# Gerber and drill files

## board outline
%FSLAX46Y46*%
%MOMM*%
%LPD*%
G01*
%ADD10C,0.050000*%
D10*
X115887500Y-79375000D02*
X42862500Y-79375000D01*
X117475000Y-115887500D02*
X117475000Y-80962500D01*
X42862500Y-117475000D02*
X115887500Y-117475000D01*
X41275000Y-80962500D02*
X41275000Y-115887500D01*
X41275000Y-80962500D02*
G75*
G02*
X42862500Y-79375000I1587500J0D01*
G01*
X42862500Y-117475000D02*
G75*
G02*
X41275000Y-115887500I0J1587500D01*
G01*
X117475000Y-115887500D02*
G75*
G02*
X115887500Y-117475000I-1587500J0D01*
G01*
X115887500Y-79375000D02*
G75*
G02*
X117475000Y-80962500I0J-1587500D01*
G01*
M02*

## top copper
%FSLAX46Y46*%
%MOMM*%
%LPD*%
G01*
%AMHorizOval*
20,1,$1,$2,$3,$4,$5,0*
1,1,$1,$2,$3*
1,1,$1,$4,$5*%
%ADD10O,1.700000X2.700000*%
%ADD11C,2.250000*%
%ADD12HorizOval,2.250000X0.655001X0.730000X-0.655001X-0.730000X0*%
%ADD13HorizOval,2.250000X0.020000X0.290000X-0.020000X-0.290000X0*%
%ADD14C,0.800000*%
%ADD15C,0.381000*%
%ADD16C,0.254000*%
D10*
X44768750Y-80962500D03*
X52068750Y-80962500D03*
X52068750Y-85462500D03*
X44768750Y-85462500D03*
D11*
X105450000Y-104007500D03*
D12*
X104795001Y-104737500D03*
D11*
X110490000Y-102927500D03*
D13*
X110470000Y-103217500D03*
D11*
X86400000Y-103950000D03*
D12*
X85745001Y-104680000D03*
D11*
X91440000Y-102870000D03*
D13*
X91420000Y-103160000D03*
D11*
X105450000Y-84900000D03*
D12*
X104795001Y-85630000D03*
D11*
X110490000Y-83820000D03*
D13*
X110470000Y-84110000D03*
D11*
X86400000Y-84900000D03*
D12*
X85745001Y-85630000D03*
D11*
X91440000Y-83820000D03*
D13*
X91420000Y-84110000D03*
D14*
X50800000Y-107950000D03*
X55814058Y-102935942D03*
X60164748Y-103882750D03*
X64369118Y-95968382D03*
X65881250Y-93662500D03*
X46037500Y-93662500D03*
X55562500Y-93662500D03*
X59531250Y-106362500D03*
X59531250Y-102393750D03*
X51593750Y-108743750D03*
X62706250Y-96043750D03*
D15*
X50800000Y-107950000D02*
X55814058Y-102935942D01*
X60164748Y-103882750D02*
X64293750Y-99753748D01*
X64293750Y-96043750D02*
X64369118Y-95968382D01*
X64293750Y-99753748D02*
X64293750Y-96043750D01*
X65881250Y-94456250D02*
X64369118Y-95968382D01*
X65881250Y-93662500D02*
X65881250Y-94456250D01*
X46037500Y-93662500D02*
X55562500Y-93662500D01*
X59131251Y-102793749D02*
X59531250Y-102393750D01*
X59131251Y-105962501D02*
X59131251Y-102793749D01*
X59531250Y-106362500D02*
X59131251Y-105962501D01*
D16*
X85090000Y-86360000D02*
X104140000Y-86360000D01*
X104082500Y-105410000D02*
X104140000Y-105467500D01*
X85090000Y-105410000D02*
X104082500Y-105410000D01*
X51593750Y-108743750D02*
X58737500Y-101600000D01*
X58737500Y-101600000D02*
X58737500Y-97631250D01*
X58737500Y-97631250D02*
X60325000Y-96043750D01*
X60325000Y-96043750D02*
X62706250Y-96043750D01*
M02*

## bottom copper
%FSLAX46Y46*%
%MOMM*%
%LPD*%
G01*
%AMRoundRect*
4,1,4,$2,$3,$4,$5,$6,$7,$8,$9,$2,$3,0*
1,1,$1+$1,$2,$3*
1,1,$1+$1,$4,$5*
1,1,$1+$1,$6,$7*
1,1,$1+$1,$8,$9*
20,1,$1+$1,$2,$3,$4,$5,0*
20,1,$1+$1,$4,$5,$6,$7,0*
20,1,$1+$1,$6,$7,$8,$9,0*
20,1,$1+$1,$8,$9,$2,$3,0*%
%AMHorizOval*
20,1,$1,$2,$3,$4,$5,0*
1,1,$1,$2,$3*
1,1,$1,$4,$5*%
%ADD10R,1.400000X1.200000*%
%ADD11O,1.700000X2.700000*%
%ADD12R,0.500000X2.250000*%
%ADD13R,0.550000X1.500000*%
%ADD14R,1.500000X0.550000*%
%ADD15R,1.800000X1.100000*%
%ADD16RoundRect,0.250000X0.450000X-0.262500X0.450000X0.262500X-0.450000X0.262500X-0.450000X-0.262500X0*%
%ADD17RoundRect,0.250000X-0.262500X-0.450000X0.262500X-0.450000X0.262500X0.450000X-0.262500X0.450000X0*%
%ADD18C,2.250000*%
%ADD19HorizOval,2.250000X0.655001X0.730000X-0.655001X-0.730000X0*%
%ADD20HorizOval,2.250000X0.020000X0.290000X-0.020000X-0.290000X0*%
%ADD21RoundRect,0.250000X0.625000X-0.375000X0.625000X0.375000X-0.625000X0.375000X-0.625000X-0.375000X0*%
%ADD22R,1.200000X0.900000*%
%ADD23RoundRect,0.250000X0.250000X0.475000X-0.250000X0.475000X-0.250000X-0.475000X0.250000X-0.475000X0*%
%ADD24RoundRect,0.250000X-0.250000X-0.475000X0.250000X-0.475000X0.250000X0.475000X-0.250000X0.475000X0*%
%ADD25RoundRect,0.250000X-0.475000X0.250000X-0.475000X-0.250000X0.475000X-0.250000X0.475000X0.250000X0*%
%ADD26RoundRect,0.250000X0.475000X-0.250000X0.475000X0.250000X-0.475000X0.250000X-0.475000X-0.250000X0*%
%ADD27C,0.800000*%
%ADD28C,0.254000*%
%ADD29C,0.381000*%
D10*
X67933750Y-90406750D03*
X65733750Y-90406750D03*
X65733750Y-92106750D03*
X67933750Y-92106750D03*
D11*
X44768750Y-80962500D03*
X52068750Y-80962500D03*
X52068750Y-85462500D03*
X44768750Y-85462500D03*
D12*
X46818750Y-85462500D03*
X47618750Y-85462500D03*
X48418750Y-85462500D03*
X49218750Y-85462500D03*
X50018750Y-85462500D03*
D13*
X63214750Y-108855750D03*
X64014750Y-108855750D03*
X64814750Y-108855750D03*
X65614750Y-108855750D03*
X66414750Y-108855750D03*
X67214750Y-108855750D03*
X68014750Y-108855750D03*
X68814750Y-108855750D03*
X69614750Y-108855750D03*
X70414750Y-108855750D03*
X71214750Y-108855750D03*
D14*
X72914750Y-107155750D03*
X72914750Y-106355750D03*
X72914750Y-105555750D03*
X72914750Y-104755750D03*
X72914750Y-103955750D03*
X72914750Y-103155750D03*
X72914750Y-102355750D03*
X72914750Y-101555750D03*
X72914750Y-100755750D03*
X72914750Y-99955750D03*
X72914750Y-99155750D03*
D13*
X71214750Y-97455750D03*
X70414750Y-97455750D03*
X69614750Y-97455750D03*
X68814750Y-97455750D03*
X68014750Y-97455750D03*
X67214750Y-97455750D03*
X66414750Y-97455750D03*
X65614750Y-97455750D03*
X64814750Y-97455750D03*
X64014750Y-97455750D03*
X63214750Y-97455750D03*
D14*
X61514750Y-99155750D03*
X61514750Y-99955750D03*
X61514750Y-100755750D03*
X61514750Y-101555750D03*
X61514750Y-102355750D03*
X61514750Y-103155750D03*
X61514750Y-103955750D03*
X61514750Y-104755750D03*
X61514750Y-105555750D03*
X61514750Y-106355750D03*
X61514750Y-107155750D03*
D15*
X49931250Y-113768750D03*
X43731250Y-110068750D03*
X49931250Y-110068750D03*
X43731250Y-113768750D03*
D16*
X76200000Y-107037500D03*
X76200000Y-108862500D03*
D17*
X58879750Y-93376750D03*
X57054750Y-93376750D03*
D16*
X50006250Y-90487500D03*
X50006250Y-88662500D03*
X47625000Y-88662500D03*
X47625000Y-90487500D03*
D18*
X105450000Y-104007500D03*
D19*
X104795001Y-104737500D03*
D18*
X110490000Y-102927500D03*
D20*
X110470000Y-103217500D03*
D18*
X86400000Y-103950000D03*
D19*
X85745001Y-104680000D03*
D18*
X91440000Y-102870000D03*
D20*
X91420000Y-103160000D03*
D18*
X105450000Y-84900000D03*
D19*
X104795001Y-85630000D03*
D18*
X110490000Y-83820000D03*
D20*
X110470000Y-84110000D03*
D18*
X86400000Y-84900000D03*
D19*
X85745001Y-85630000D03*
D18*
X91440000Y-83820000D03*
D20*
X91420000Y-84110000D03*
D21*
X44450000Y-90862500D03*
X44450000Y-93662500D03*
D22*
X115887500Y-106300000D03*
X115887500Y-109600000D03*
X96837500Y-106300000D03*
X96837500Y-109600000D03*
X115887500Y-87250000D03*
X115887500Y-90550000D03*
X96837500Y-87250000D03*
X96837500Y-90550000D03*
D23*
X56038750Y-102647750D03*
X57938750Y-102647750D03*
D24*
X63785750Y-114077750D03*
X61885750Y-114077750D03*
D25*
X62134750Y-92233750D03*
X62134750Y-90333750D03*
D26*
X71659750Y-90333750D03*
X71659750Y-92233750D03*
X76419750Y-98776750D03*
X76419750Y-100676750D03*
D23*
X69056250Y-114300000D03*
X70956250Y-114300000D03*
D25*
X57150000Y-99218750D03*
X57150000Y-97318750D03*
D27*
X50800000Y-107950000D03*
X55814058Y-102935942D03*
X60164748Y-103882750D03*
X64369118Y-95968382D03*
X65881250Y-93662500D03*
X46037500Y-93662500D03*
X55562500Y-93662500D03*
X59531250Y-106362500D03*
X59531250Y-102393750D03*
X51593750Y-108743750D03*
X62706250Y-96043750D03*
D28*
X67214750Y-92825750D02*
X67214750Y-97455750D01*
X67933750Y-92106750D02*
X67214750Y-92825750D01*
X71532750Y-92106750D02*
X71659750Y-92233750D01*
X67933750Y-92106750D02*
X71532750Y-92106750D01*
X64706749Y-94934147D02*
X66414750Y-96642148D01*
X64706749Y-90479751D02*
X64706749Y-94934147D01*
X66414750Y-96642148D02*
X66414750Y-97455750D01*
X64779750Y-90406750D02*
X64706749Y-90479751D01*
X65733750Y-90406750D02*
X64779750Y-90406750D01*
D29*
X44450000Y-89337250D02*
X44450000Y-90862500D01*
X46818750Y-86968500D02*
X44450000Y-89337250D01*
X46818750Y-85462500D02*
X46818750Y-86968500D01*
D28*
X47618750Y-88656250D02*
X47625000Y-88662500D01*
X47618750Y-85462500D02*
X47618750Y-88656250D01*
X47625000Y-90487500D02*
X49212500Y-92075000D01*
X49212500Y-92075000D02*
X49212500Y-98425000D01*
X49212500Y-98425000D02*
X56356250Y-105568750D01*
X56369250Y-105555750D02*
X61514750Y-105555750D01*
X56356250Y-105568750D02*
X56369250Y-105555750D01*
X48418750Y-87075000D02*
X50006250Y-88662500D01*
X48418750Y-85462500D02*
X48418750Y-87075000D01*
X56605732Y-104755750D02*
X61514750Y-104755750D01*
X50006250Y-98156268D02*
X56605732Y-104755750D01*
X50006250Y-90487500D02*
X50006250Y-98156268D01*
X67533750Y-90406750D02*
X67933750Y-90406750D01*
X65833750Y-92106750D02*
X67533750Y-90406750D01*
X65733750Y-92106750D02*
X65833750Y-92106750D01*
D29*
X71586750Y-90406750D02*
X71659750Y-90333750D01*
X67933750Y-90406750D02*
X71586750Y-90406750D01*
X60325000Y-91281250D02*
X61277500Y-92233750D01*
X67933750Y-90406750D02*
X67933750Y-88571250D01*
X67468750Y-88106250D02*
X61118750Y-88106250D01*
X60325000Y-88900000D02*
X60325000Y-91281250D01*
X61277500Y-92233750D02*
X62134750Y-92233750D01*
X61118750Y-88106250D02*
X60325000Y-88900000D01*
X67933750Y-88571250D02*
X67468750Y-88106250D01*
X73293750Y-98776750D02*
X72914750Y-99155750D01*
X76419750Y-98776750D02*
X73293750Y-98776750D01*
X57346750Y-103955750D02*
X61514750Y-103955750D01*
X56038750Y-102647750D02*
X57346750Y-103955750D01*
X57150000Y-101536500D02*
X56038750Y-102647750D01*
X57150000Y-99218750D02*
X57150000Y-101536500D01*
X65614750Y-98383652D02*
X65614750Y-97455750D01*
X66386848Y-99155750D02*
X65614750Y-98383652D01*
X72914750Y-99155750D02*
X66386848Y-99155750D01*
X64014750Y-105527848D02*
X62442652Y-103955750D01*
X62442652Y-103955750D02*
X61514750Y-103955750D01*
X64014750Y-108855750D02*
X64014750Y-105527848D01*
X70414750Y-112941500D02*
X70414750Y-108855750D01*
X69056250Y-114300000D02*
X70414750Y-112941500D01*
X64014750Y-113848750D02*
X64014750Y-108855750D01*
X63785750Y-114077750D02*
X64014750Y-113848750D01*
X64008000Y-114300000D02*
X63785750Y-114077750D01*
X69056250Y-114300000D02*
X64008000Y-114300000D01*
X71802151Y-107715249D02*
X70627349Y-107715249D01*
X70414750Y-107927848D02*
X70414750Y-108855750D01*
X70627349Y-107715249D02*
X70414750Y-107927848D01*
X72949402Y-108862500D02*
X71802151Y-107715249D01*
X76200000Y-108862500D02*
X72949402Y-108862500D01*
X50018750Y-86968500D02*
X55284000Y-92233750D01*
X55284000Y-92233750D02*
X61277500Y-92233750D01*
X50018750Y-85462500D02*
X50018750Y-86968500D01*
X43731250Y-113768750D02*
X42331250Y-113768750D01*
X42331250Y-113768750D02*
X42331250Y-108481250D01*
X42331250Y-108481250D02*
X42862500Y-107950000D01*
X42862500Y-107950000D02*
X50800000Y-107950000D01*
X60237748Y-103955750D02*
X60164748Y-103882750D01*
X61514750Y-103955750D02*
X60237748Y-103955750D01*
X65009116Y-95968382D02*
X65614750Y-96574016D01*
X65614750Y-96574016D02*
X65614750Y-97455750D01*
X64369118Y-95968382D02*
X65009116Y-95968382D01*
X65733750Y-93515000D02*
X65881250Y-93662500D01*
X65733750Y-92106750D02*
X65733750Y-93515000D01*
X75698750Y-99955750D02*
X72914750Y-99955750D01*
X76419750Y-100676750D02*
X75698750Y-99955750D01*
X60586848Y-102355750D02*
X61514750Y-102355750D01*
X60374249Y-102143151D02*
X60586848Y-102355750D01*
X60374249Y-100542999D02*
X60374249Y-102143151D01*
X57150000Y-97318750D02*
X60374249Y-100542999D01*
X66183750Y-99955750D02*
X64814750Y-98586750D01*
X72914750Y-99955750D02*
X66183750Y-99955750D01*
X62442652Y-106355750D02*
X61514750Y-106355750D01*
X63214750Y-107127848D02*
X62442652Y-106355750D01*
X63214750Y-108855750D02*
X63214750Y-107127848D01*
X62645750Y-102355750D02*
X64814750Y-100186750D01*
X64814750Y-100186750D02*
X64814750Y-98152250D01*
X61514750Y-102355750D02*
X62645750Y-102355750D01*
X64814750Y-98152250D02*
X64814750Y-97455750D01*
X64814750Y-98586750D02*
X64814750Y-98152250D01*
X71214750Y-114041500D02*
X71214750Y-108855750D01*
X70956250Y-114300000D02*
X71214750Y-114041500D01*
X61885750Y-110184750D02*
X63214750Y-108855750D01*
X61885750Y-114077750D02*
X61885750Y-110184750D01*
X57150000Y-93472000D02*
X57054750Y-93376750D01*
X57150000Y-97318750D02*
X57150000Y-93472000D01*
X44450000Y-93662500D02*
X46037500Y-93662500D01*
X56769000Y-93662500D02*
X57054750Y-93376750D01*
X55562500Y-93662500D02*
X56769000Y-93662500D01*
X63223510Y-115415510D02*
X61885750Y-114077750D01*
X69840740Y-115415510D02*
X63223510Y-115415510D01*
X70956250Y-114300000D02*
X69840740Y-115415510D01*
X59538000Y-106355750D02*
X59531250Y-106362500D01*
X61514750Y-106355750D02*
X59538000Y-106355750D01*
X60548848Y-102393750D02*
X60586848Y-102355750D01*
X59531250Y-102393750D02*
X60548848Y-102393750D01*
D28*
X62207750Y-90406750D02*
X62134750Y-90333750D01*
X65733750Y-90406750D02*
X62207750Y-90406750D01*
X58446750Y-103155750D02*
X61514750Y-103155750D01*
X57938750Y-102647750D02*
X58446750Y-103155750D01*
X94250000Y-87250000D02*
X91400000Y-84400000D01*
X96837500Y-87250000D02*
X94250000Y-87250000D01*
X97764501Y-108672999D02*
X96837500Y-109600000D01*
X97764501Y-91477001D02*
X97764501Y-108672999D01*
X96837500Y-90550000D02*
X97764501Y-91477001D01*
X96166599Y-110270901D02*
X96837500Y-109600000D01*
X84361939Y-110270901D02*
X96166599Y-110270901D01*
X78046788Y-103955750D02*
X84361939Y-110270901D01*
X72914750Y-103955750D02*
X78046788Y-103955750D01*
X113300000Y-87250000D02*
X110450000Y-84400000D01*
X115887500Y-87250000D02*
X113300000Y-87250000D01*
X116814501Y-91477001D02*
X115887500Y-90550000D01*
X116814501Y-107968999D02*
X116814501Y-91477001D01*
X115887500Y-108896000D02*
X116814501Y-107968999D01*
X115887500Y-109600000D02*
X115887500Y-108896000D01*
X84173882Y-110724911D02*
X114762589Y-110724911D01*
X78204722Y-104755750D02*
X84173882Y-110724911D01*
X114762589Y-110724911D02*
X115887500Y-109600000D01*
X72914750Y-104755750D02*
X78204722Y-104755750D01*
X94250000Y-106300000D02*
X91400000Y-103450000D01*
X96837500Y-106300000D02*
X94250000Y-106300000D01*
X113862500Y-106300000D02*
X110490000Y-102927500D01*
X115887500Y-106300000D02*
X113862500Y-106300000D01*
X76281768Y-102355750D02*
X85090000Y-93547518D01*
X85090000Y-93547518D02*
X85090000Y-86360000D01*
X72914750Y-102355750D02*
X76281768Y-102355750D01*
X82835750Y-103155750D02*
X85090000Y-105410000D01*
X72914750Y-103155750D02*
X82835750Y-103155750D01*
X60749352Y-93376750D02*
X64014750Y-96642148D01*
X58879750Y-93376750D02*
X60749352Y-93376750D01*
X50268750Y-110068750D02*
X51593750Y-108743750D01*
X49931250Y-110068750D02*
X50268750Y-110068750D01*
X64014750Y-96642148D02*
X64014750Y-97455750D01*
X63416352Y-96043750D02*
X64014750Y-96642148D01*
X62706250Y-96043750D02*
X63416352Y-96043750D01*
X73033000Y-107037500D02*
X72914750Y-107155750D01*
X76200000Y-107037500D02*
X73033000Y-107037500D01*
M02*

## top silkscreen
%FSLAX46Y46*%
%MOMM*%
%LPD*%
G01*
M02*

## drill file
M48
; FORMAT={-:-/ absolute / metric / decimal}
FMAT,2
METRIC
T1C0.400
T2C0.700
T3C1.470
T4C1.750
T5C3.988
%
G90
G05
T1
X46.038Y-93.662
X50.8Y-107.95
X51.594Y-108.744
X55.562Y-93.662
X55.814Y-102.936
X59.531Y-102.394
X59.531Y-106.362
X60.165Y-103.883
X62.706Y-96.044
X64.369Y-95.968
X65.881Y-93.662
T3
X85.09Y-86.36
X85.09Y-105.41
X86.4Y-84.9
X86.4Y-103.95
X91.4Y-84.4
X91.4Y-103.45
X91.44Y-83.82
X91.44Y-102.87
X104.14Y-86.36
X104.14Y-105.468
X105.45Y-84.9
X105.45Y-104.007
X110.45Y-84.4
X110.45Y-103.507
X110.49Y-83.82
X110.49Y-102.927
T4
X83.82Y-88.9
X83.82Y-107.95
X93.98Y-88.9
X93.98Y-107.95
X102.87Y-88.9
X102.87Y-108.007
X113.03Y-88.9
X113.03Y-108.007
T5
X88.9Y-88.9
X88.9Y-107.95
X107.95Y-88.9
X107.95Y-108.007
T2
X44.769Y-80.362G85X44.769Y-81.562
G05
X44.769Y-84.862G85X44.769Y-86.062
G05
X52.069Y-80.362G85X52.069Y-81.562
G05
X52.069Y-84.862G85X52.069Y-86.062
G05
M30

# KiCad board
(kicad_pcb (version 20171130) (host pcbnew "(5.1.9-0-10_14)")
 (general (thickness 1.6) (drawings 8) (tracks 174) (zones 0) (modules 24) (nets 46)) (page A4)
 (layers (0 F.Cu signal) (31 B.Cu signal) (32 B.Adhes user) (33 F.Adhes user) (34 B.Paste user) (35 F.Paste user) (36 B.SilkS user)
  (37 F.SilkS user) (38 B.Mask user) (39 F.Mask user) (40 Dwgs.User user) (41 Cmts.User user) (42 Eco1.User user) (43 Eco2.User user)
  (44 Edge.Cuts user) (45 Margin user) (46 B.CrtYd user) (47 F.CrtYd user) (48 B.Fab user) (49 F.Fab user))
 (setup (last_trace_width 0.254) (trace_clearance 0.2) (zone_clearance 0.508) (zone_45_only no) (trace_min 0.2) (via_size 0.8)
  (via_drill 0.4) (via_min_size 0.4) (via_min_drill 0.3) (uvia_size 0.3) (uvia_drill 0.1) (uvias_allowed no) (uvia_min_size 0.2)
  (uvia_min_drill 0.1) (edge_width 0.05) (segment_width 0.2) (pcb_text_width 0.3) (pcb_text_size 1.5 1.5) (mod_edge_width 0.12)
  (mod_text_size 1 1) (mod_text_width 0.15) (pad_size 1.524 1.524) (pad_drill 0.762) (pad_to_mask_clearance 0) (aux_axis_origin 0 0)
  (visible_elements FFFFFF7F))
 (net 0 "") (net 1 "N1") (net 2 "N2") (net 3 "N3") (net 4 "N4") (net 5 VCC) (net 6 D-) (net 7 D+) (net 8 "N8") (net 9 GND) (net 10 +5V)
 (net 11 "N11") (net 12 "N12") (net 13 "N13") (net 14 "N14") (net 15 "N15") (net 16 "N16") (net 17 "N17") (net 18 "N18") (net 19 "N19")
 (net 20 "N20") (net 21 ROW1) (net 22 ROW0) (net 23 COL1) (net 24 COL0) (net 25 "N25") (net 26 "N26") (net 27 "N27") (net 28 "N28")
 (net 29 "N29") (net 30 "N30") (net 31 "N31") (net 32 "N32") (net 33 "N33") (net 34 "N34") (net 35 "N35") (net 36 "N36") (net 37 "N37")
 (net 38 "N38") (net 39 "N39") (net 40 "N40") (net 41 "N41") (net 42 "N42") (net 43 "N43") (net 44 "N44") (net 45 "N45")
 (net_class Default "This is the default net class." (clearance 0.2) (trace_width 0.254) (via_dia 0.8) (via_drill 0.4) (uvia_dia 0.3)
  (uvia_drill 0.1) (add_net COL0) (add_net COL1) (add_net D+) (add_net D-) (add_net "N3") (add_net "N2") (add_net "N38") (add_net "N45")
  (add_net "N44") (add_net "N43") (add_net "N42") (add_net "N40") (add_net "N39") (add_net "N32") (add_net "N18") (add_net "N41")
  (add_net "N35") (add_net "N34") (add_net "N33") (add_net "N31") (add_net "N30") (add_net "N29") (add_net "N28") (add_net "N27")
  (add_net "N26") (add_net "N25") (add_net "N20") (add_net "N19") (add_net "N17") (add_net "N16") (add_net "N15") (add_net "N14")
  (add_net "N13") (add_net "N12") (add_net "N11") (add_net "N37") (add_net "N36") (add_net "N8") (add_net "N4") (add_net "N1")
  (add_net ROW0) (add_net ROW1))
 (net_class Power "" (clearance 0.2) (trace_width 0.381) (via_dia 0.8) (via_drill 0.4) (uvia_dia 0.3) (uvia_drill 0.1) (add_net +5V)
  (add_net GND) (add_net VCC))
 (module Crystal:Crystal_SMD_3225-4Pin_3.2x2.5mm (layer B.Cu) (at 66.83375 91.25675 180)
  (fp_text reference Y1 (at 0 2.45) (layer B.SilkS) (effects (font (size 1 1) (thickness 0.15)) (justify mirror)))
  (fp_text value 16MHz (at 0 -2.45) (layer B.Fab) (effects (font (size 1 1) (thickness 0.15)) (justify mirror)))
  (pad 4 smd rect (at -1.1 0.85 180) (size 1.4 1.2) (layers B.Cu B.Paste B.Mask) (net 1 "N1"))
  (pad 3 smd rect (at 1.1 0.85 180) (size 1.4 1.2) (layers B.Cu B.Paste B.Mask) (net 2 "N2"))
  (pad 2 smd rect (at 1.1 -0.85 180) (size 1.4 1.2) (layers B.Cu B.Paste B.Mask) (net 1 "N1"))
  (pad 1 smd rect (at -1.1 -0.85 180) (size 1.4 1.2) (layers B.Cu B.Paste B.Mask) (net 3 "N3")))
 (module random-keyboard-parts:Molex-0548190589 (layer B.Cu) (at 48.41875 80.9625 270)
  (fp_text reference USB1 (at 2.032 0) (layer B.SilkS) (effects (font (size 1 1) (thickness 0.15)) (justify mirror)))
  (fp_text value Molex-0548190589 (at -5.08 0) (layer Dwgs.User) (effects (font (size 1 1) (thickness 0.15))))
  (pad 6 thru_hole oval (at 0 3.65 270) (size 2.7 1.7) (drill oval 1.9 0.7) (layers *.Cu *.Mask) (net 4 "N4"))
  (pad 6 thru_hole oval (at 0 -3.65 270) (size 2.7 1.7) (drill oval 1.9 0.7) (layers *.Cu *.Mask) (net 4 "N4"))
  (pad 6 thru_hole oval (at 4.5 -3.65 270) (size 2.7 1.7) (drill oval 1.9 0.7) (layers *.Cu *.Mask) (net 4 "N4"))
  (pad 6 thru_hole oval (at 4.5 3.65 270) (size 2.7 1.7) (drill oval 1.9 0.7) (layers *.Cu *.Mask) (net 4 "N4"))
  (pad 5 smd rect (at 4.5 1.6 270) (size 2.25 0.5) (layers B.Cu B.Paste B.Mask) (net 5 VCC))
  (pad 4 smd rect (at 4.5 0.8 270) (size 2.25 0.5) (layers B.Cu B.Paste B.Mask) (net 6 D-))
  (pad 3 smd rect (at 4.5 0 270) (size 2.25 0.5) (layers B.Cu B.Paste B.Mask) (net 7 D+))
  (pad 2 smd rect (at 4.5 -0.8 270) (size 2.25 0.5) (layers B.Cu B.Paste B.Mask) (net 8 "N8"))
  (pad 1 smd rect (at 4.5 -1.6 270) (size 2.25 0.5) (layers B.Cu B.Paste B.Mask) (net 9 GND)))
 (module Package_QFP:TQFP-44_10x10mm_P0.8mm (layer B.Cu) (at 67.21475 103.15575)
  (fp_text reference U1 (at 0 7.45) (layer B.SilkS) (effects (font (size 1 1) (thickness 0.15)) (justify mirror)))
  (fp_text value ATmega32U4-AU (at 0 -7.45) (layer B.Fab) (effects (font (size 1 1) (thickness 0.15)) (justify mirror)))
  (pad 44 smd rect (at -4 5.7 270) (size 1.5 0.55) (layers B.Cu B.Paste B.Mask) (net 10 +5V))
  (pad 43 smd rect (at -3.2 5.7 270) (size 1.5 0.55) (layers B.Cu B.Paste B.Mask) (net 9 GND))
  (pad 42 smd rect (at -2.4 5.7 270) (size 1.5 0.55) (layers B.Cu B.Paste B.Mask) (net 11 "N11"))
  (pad 41 smd rect (at -1.6 5.7 270) (size 1.5 0.55) (layers B.Cu B.Paste B.Mask) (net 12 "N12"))
  (pad 40 smd rect (at -0.8 5.7 270) (size 1.5 0.55) (layers B.Cu B.Paste B.Mask) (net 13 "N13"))
  (pad 39 smd rect (at 0 5.7 270) (size 1.5 0.55) (layers B.Cu B.Paste B.Mask) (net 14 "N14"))
  (pad 38 smd rect (at 0.8 5.7 270) (size 1.5 0.55) (layers B.Cu B.Paste B.Mask) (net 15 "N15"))
  (pad 37 smd rect (at 1.6 5.7 270) (size 1.5 0.55) (layers B.Cu B.Paste B.Mask) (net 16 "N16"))
  (pad 36 smd rect (at 2.4 5.7 270) (size 1.5 0.55) (layers B.Cu B.Paste B.Mask) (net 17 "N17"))
  (pad 35 smd rect (at 3.2 5.7 270) (size 1.5 0.55) (layers B.Cu B.Paste B.Mask) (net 9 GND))
  (pad 34 smd rect (at 4 5.7 270) (size 1.5 0.55) (layers B.Cu B.Paste B.Mask) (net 10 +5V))
  (pad 33 smd rect (at 5.7 4) (size 1.5 0.55) (layers B.Cu B.Paste B.Mask) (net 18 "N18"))
  (pad 32 smd rect (at 5.7 3.2) (size 1.5 0.55) (layers B.Cu B.Paste B.Mask) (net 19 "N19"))
  (pad 31 smd rect (at 5.7 2.4) (size 1.5 0.55) (layers B.Cu B.Paste B.Mask) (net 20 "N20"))
  (pad 30 smd rect (at 5.7 1.6) (size 1.5 0.55) (layers B.Cu B.Paste B.Mask) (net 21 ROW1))
  (pad 29 smd rect (at 5.7 0.8) (size 1.5 0.55) (layers B.Cu B.Paste B.Mask) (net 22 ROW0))
  (pad 28 smd rect (at 5.7 0) (size 1.5 0.55) (layers B.Cu B.Paste B.Mask) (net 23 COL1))
  (pad 27 smd rect (at 5.7 -0.8) (size 1.5 0.55) (layers B.Cu B.Paste B.Mask) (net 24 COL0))
  (pad 26 smd rect (at 5.7 -1.6) (size 1.5 0.55) (layers B.Cu B.Paste B.Mask) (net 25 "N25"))
  (pad 25 smd rect (at 5.7 -2.4) (size 1.5 0.55) (layers B.Cu B.Paste B.Mask) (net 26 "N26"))
  (pad 24 smd rect (at 5.7 -3.2) (size 1.5 0.55) (layers B.Cu B.Paste B.Mask) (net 10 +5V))
  (pad 23 smd rect (at 5.7 -4) (size 1.5 0.55) (layers B.Cu B.Paste B.Mask) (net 9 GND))
  (pad 22 smd rect (at 4 -5.7 270) (size 1.5 0.55) (layers B.Cu B.Paste B.Mask) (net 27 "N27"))
  (pad 21 smd rect (at 3.2 -5.7 270) (size 1.5 0.55) (layers B.Cu B.Paste B.Mask) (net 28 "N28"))
  (pad 20 smd rect (at 2.4 -5.7 270) (size 1.5 0.55) (layers B.Cu B.Paste B.Mask) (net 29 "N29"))
  (pad 19 smd rect (at 1.6 -5.7 270) (size 1.5 0.55) (layers B.Cu B.Paste B.Mask) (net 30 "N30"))
  (pad 18 smd rect (at 0.8 -5.7 270) (size 1.5 0.55) (layers B.Cu B.Paste B.Mask) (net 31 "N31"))
  (pad 17 smd rect (at 0 -5.7 270) (size 1.5 0.55) (layers B.Cu B.Paste B.Mask) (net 3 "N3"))
  (pad 16 smd rect (at -0.8 -5.7 270) (size 1.5 0.55) (layers B.Cu B.Paste B.Mask) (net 2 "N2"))
  (pad 15 smd rect (at -1.6 -5.7 270) (size 1.5 0.55) (layers B.Cu B.Paste B.Mask) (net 9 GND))
  (pad 14 smd rect (at -2.4 -5.7 270) (size 1.5 0.55) (layers B.Cu B.Paste B.Mask) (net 10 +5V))
  (pad 13 smd rect (at -3.2 -5.7 270) (size 1.5 0.55) (layers B.Cu B.Paste B.Mask) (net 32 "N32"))
  (pad 12 smd rect (at -4 -5.7 270) (size 1.5 0.55) (layers B.Cu B.Paste B.Mask) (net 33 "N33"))
  (pad 11 smd rect (at -5.7 -4) (size 1.5 0.55) (layers B.Cu B.Paste B.Mask) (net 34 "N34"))
  (pad 10 smd rect (at -5.7 -3.2) (size 1.5 0.55) (layers B.Cu B.Paste B.Mask) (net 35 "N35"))
  (pad 9 smd rect (at -5.7 -2.4) (size 1.5 0.55) (layers B.Cu B.Paste B.Mask) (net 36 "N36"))
  (pad 8 smd rect (at -5.7 -1.6) (size 1.5 0.55) (layers B.Cu B.Paste B.Mask) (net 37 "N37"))
  (pad 7 smd rect (at -5.7 -0.8) (size 1.5 0.55) (layers B.Cu B.Paste B.Mask) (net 10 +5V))
  (pad 6 smd rect (at -5.7 0) (size 1.5 0.55) (layers B.Cu B.Paste B.Mask) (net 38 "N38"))
  (pad 5 smd rect (at -5.7 0.8) (size 1.5 0.55) (layers B.Cu B.Paste B.Mask) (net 9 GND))
  (pad 4 smd rect (at -5.7 1.6) (size 1.5 0.55) (layers B.Cu B.Paste B.Mask) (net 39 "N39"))
  (pad 3 smd rect (at -5.7 2.4) (size 1.5 0.55) (layers B.Cu B.Paste B.Mask) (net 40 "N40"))
  (pad 2 smd rect (at -5.7 3.2) (size 1.5 0.55) (layers B.Cu B.Paste B.Mask) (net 10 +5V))
  (pad 1 smd rect (at -5.7 4) (size 1.5 0.55) (layers B.Cu B.Paste B.Mask) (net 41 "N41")))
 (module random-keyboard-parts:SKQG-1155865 (layer B.Cu) (at 46.83125 111.91875 180)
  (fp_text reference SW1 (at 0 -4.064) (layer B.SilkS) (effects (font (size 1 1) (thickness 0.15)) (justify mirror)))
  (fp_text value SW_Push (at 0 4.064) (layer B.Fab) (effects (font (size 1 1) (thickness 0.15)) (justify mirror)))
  (pad 4 smd rect (at -3.1 -1.85 180) (size 1.8 1.1) (layers B.Cu B.Paste B.Mask))
  (pad 3 smd rect (at 3.1 1.85 180) (size 1.8 1.1) (layers B.Cu B.Paste B.Mask))
  (pad 2 smd rect (at -3.1 1.85 180) (size 1.8 1.1) (layers B.Cu B.Paste B.Mask) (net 32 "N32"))
  (pad 1 smd rect (at 3.1 -1.85 180) (size 1.8 1.1) (layers B.Cu B.Paste B.Mask) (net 9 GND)))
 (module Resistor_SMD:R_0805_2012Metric (layer B.Cu) (at 76.2 107.95 90)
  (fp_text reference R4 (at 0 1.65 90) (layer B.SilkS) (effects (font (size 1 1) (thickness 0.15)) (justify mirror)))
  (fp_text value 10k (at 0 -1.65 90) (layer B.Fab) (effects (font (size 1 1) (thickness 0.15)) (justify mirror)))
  (pad 2 smd roundrect (at 0.9125 0 90) (size 1.025 1.4) (layers B.Cu B.Paste B.Mask) (roundrect_rratio 0.243902) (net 18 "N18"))
  (pad 1 smd roundrect (at -0.9125 0 90) (size 1.025 1.4) (layers B.Cu B.Paste B.Mask) (roundrect_rratio 0.243902) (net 9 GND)))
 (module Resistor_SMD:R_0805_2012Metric (layer B.Cu) (at 57.96725 93.37675)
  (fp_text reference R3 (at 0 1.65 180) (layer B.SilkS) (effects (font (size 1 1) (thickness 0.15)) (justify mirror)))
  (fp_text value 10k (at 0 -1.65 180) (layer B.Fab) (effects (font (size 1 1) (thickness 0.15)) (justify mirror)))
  (pad 2 smd roundrect (at 0.9125 0) (size 1.025 1.4) (layers B.Cu B.Paste B.Mask) (roundrect_rratio 0.243902) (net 32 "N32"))
  (pad 1 smd roundrect (at -0.9125 0) (size 1.025 1.4) (layers B.Cu B.Paste B.Mask) (roundrect_rratio 0.243902) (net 10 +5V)))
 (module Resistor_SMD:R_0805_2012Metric (layer B.Cu) (at 50.00625 89.575 90)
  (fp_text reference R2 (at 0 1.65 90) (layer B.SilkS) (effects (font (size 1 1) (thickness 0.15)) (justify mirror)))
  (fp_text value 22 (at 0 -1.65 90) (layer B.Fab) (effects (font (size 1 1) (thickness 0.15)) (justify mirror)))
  (pad 1 smd roundrect (at -0.9125 0 90) (size 1.025 1.4) (layers B.Cu B.Paste B.Mask) (roundrect_rratio 0.243902) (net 39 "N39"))
  (pad 2 smd roundrect (at 0.9125 0 90) (size 1.025 1.4) (layers B.Cu B.Paste B.Mask) (roundrect_rratio 0.243902) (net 7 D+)))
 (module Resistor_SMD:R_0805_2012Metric (layer B.Cu) (at 47.625 89.575 90)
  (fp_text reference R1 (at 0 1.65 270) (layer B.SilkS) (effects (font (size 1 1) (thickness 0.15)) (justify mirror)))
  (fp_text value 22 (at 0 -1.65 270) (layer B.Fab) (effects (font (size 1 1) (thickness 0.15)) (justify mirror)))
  (pad 2 smd roundrect (at 0.9125 0 90) (size 1.025 1.4) (layers B.Cu B.Paste B.Mask) (roundrect_rratio 0.243902) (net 6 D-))
  (pad 1 smd roundrect (at -0.9125 0 90) (size 1.025 1.4) (layers B.Cu B.Paste B.Mask) (roundrect_rratio 0.243902) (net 40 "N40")))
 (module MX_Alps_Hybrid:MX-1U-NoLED (layer F.Cu) (at 107.95 108.0075)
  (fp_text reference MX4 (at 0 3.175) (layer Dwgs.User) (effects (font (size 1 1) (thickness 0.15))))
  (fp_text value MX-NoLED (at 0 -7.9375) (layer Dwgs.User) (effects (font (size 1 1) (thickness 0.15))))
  (pad "" np_thru_hole circle (at 5.08 0 48.0996) (size 1.75 1.75) (drill 1.75) (layers *.Cu *.Mask))
  (pad "" np_thru_hole circle (at -5.08 0 48.0996) (size 1.75 1.75) (drill 1.75) (layers *.Cu *.Mask))
  (pad 1 thru_hole circle (at -2.5 -4) (size 2.25 2.25) (drill 1.47) (layers *.Cu B.Mask) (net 23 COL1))
  (pad "" np_thru_hole circle (at 0 0) (size 3.9878 3.9878) (drill 3.9878) (layers *.Cu *.Mask))
  (pad 1 thru_hole oval (at -3.81 -2.54 48.0996) (size 4.211556 2.25) (drill 1.47 (offset 0.980778 0)) (layers *.Cu B.Mask) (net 23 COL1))
  (pad 2 thru_hole circle (at 2.54 -5.08) (size 2.25 2.25) (drill 1.47) (layers *.Cu B.Mask) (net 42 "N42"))
  (pad 2 thru_hole oval (at 2.5 -4.5 86.0548) (size 2.831378 2.25) (drill 1.47 (offset 0.290689 0)) (layers *.Cu B.Mask) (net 42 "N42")))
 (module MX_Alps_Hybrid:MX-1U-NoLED (layer F.Cu) (at 88.9 107.95)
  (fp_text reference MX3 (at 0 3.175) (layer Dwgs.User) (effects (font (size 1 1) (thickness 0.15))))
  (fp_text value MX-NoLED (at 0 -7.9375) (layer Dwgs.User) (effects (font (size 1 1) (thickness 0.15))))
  (pad "" np_thru_hole circle (at 5.08 0 48.0996) (size 1.75 1.75) (drill 1.75) (layers *.Cu *.Mask))
  (pad "" np_thru_hole circle (at -5.08 0 48.0996) (size 1.75 1.75) (drill 1.75) (layers *.Cu *.Mask))
  (pad 1 thru_hole circle (at -2.5 -4) (size 2.25 2.25) (drill 1.47) (layers *.Cu B.Mask) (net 23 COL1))
  (pad "" np_thru_hole circle (at 0 0) (size 3.9878 3.9878) (drill 3.9878) (layers *.Cu *.Mask))
  (pad 1 thru_hole oval (at -3.81 -2.54 48.0996) (size 4.211556 2.25) (drill 1.47 (offset 0.980778 0)) (layers *.Cu B.Mask) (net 23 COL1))
  (pad 2 thru_hole circle (at 2.54 -5.08) (size 2.25 2.25) (drill 1.47) (layers *.Cu B.Mask) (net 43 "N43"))
  (pad 2 thru_hole oval (at 2.5 -4.5 86.0548) (size 2.831378 2.25) (drill 1.47 (offset 0.290689 0)) (layers *.Cu B.Mask) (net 43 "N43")))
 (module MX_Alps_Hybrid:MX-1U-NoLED (layer F.Cu) (at 107.95 88.9)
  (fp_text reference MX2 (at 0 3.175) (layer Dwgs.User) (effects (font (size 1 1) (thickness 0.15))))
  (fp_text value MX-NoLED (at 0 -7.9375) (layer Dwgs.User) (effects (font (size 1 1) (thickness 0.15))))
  (pad "" np_thru_hole circle (at 5.08 0 48.0996) (size 1.75 1.75) (drill 1.75) (layers *.Cu *.Mask))
  (pad "" np_thru_hole circle (at -5.08 0 48.0996) (size 1.75 1.75) (drill 1.75) (layers *.Cu *.Mask))
  (pad 1 thru_hole circle (at -2.5 -4) (size 2.25 2.25) (drill 1.47) (layers *.Cu B.Mask) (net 24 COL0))
  (pad "" np_thru_hole circle (at 0 0) (size 3.9878 3.9878) (drill 3.9878) (layers *.Cu *.Mask))
  (pad 1 thru_hole oval (at -3.81 -2.54 48.0996) (size 4.211556 2.25) (drill 1.47 (offset 0.980778 0)) (layers *.Cu B.Mask) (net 24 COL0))
  (pad 2 thru_hole circle (at 2.54 -5.08) (size 2.25 2.25) (drill 1.47) (layers *.Cu B.Mask) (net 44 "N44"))
  (pad 2 thru_hole oval (at 2.5 -4.5 86.0548) (size 2.831378 2.25) (drill 1.47 (offset 0.290689 0)) (layers *.Cu B.Mask) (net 44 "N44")))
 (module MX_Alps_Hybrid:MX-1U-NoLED (layer F.Cu) (at 88.9 88.9)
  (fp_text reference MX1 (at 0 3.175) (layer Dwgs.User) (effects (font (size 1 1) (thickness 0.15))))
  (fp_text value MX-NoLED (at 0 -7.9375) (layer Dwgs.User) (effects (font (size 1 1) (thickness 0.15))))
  (pad "" np_thru_hole circle (at 5.08 0 48.0996) (size 1.75 1.75) (drill 1.75) (layers *.Cu *.Mask))
  (pad "" np_thru_hole circle (at -5.08 0 48.0996) (size 1.75 1.75) (drill 1.75) (layers *.Cu *.Mask))
  (pad 1 thru_hole circle (at -2.5 -4) (size 2.25 2.25) (drill 1.47) (layers *.Cu B.Mask) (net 24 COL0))
  (pad "" np_thru_hole circle (at 0 0) (size 3.9878 3.9878) (drill 3.9878) (layers *.Cu *.Mask))
  (pad 1 thru_hole oval (at -3.81 -2.54 48.0996) (size 4.211556 2.25) (drill 1.47 (offset 0.980778 0)) (layers *.Cu B.Mask) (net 24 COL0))
  (pad 2 thru_hole circle (at 2.54 -5.08) (size 2.25 2.25) (drill 1.47) (layers *.Cu B.Mask) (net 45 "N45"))
  (pad 2 thru_hole oval (at 2.5 -4.5 86.0548) (size 2.831378 2.25) (drill 1.47 (offset 0.290689 0)) (layers *.Cu B.Mask) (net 45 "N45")))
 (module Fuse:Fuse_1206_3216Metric (layer B.Cu) (at 44.45 92.2625 90)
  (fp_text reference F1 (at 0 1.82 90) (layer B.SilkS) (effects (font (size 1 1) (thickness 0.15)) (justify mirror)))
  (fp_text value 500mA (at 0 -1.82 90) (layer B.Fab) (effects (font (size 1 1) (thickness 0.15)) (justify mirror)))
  (pad 2 smd roundrect (at 1.4 0 90) (size 1.25 1.75) (layers B.Cu B.Paste B.Mask) (roundrect_rratio 0.2) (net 5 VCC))
  (pad 1 smd roundrect (at -1.4 0 90) (size 1.25 1.75) (layers B.Cu B.Paste B.Mask) (roundrect_rratio 0.2) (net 10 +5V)))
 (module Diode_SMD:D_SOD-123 (layer B.Cu) (at 115.8875 107.95 90)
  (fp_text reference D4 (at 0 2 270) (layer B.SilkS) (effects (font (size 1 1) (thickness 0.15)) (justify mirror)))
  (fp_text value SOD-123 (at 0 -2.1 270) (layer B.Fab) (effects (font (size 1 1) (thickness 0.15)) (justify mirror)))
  (pad 2 smd rect (at 1.65 0 90) (size 0.9 1.2) (layers B.Cu B.Paste B.Mask) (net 42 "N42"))
  (pad 1 smd rect (at -1.65 0 90) (size 0.9 1.2) (layers B.Cu B.Paste B.Mask) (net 21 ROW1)))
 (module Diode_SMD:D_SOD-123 (layer B.Cu) (at 96.8375 107.95 90)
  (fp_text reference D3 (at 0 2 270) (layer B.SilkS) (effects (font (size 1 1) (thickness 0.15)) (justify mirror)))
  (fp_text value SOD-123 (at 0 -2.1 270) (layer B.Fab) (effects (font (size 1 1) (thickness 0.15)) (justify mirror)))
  (pad 2 smd rect (at 1.65 0 90) (size 0.9 1.2) (layers B.Cu B.Paste B.Mask) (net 43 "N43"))
  (pad 1 smd rect (at -1.65 0 90) (size 0.9 1.2) (layers B.Cu B.Paste B.Mask) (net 22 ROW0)))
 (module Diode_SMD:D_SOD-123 (layer B.Cu) (at 115.8875 88.9 90)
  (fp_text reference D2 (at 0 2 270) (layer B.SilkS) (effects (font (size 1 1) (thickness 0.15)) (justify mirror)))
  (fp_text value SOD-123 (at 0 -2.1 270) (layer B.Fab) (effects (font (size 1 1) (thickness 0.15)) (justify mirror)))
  (pad 2 smd rect (at 1.65 0 90) (size 0.9 1.2) (layers B.Cu B.Paste B.Mask) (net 44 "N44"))
  (pad 1 smd rect (at -1.65 0 90) (size 0.9 1.2) (layers B.Cu B.Paste B.Mask) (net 21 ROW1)))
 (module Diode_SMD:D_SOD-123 (layer B.Cu) (at 96.8375 88.9 90)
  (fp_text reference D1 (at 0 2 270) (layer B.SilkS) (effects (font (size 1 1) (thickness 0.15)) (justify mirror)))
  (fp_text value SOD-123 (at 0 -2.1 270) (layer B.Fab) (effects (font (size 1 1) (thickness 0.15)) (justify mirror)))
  (pad 2 smd rect (at 1.65 0 90) (size 0.9 1.2) (layers B.Cu B.Paste B.Mask) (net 45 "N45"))
  (pad 1 smd rect (at -1.65 0 90) (size 0.9 1.2) (layers B.Cu B.Paste B.Mask) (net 22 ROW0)))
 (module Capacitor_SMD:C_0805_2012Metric (layer B.Cu) (at 56.98875 102.64775 180)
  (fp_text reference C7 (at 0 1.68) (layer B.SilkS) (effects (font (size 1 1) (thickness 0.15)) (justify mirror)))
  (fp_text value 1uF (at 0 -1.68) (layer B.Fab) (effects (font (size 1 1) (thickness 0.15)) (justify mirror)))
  (pad 2 smd roundrect (at 0.95 0 180) (size 1 1.45) (layers B.Cu B.Paste B.Mask) (roundrect_rratio 0.25) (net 9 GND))
  (pad 1 smd roundrect (at -0.95 0 180) (size 1 1.45) (layers B.Cu B.Paste B.Mask) (roundrect_rratio 0.25) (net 38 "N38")))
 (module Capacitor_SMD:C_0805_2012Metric (layer B.Cu) (at 62.83575 114.07775)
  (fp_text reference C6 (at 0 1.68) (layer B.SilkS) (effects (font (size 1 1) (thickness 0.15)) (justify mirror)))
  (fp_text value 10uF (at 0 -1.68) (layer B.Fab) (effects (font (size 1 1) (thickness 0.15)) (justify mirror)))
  (pad 2 smd roundrect (at 0.95 0) (size 1 1.45) (layers B.Cu B.Paste B.Mask) (roundrect_rratio 0.25) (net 9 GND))
  (pad 1 smd roundrect (at -0.95 0) (size 1 1.45) (layers B.Cu B.Paste B.Mask) (roundrect_rratio 0.25) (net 10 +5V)))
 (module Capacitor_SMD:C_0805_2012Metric (layer B.Cu) (at 62.13475 91.28375 270)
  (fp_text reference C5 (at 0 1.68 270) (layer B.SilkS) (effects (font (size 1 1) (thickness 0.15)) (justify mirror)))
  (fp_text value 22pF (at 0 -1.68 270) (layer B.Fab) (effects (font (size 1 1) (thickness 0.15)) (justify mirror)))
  (pad 2 smd roundrect (at 0.95 0 270) (size 1 1.45) (layers B.Cu B.Paste B.Mask) (roundrect_rratio 0.25) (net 9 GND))
  (pad 1 smd roundrect (at -0.95 0 270) (size 1 1.45) (layers B.Cu B.Paste B.Mask) (roundrect_rratio 0.25) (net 2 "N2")))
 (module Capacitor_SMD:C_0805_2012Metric (layer B.Cu) (at 71.65975 91.28375 90)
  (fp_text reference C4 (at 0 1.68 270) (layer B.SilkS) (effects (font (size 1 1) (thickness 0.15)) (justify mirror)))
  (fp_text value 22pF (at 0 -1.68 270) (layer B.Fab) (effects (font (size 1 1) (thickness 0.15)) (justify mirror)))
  (pad 2 smd roundrect (at 0.95 0 90) (size 1 1.45) (layers B.Cu B.Paste B.Mask) (roundrect_rratio 0.25) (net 9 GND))
  (pad 1 smd roundrect (at -0.95 0 90) (size 1 1.45) (layers B.Cu B.Paste B.Mask) (roundrect_rratio 0.25) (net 3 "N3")))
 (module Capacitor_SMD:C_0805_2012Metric (layer B.Cu) (at 76.41975 99.72675 90)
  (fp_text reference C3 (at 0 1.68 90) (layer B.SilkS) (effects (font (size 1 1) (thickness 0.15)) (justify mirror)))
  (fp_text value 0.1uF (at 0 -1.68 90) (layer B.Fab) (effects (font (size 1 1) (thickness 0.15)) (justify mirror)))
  (pad 2 smd roundrect (at 0.95 0 90) (size 1 1.45) (layers B.Cu B.Paste B.Mask) (roundrect_rratio 0.25) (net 9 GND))
  (pad 1 smd roundrect (at -0.95 0 90) (size 1 1.45) (layers B.Cu B.Paste B.Mask) (roundrect_rratio 0.25) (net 10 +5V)))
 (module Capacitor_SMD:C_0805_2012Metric (layer B.Cu) (at 70.00625 114.3 180)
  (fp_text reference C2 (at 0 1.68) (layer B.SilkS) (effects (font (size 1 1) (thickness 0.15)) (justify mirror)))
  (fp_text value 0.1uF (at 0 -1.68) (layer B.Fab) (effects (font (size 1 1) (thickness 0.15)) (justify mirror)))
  (pad 2 smd roundrect (at 0.95 0 180) (size 1 1.45) (layers B.Cu B.Paste B.Mask) (roundrect_rratio 0.25) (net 9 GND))
  (pad 1 smd roundrect (at -0.95 0 180) (size 1 1.45) (layers B.Cu B.Paste B.Mask) (roundrect_rratio 0.25) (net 10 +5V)))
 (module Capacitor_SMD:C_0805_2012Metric (layer B.Cu) (at 57.15 98.26875 270)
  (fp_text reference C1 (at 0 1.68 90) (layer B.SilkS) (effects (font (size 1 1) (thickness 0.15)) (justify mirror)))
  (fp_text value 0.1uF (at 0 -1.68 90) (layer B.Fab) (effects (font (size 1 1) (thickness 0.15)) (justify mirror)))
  (pad 2 smd roundrect (at 0.95 0 270) (size 1 1.45) (layers B.Cu B.Paste B.Mask) (roundrect_rratio 0.25) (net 9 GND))
  (pad 1 smd roundrect (at -0.95 0 270) (size 1 1.45) (layers B.Cu B.Paste B.Mask) (roundrect_rratio 0.25) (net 10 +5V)))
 (gr_line (start 115.8875 79.375) (end 42.8625 79.375) (layer Edge.Cuts) (width 0.05))
 (gr_line (start 117.475 115.8875) (end 117.475 80.9625) (layer Edge.Cuts) (width 0.05))
 (gr_line (start 42.8625 117.475) (end 115.8875 117.475) (layer Edge.Cuts) (width 0.05))
 (gr_line (start 41.275 80.9625) (end 41.275 115.8875) (layer Edge.Cuts) (width 0.05))
 (gr_arc (start 42.8625 80.9625) (end 42.8625 79.375) (angle -90) (layer Edge.Cuts) (width 0.05))
 (gr_arc (start 42.8625 115.8875) (end 41.275 115.8875) (angle -90) (layer Edge.Cuts) (width 0.05))
 (gr_arc (start 115.8875 115.8875) (end 115.8875 117.475) (angle -90) (layer Edge.Cuts) (width 0.05))
 (gr_arc (start 115.8875 80.9625) (end 117.475 80.9625) (angle -90) (layer Edge.Cuts) (width 0.05))
 (segment (start 67.21475 92.82575) (end 67.21475 97.45575) (width 0.254) (layer B.Cu) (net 3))
 (segment (start 67.93375 92.10675) (end 67.21475 92.82575) (width 0.254) (layer B.Cu) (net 3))
 (segment (start 71.53275 92.10675) (end 71.65975 92.23375) (width 0.254) (layer B.Cu) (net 3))
 (segment (start 67.93375 92.10675) (end 71.53275 92.10675) (width 0.254) (layer B.Cu) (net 3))
 (segment (start 64.706749 94.934147) (end 66.41475 96.642148) (width 0.254) (layer B.Cu) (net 2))
 (segment (start 64.706749 90.479751) (end 64.706749 94.934147) (width 0.254) (layer B.Cu) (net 2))
 (segment (start 66.41475 96.642148) (end 66.41475 97.45575) (width 0.254) (layer B.Cu) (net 2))
 (segment (start 64.77975 90.40675) (end 64.706749 90.479751) (width 0.254) (layer B.Cu) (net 2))
 (segment (start 65.73375 90.40675) (end 64.77975 90.40675) (width 0.254) (layer B.Cu) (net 2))
 (segment (start 44.45 89.33725) (end 44.45 90.8625) (width 0.381) (layer B.Cu) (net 5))
 (segment (start 46.81875 86.9685) (end 44.45 89.33725) (width 0.381) (layer B.Cu) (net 5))
 (segment (start 46.81875 85.4625) (end 46.81875 86.9685) (width 0.381) (layer B.Cu) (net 5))
 (segment (start 47.61875 88.65625) (end 47.625 88.6625) (width 0.254) (layer B.Cu) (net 6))
 (segment (start 47.61875 85.4625) (end 47.61875 88.65625) (width 0.254) (layer B.Cu) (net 6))
 (segment (start 47.625 90.4875) (end 49.2125 92.075) (width 0.254) (layer B.Cu) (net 40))
 (segment (start 49.2125 92.075) (end 49.2125 98.425) (width 0.254) (layer B.Cu) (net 40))
 (segment (start 49.2125 98.425) (end 56.35625 105.56875) (width 0.254) (layer B.Cu) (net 40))
 (segment (start 56.36925 105.55575) (end 61.51475 105.55575) (width 0.254) (layer B.Cu) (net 40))
 (segment (start 56.35625 105.56875) (end 56.36925 105.55575) (width 0.254) (layer B.Cu) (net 40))
 (segment (start 48.41875 87.075) (end 50.00625 88.6625) (width 0.254) (layer B.Cu) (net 7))
 (segment (start 48.41875 85.4625) (end 48.41875 87.075) (width 0.254) (layer B.Cu) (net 7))
 (segment (start 56.605732 104.75575) (end 61.51475 104.75575) (width 0.254) (layer B.Cu) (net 39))
 (segment (start 50.00625 98.156268) (end 56.605732 104.75575) (width 0.254) (layer B.Cu) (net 39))
 (segment (start 50.00625 90.4875) (end 50.00625 98.156268) (width 0.254) (layer B.Cu) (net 39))
 (segment (start 67.53375 90.40675) (end 67.93375 90.40675) (width 0.254) (layer B.Cu) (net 9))
 (segment (start 65.83375 92.10675) (end 67.53375 90.40675) (width 0.254) (layer B.Cu) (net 9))
 (segment (start 65.73375 92.10675) (end 65.83375 92.10675) (width 0.254) (layer B.Cu) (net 9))
 (segment (start 71.58675 90.40675) (end 71.65975 90.33375) (width 0.381) (layer B.Cu) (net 9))
 (segment (start 67.93375 90.40675) (end 71.58675 90.40675) (width 0.381) (layer B.Cu) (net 9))
 (segment (start 60.325 91.28125) (end 61.2775 92.23375) (width 0.381) (layer B.Cu) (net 9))
 (segment (start 67.93375 90.40675) (end 67.93375 88.57125) (width 0.381) (layer B.Cu) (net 9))
 (segment (start 67.46875 88.10625) (end 61.11875 88.10625) (width 0.381) (layer B.Cu) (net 9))
 (segment (start 60.325 88.9) (end 60.325 91.28125) (width 0.381) (layer B.Cu) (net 9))
 (segment (start 61.2775 92.23375) (end 62.13475 92.23375) (width 0.381) (layer B.Cu) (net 9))
 (segment (start 61.11875 88.10625) (end 60.325 88.9) (width 0.381) (layer B.Cu) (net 9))
 (segment (start 67.93375 88.57125) (end 67.46875 88.10625) (width 0.381) (layer B.Cu) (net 9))
 (segment (start 73.29375 98.77675) (end 72.91475 99.15575) (width 0.381) (layer B.Cu) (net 9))
 (segment (start 76.41975 98.77675) (end 73.29375 98.77675) (width 0.381) (layer B.Cu) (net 9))
 (segment (start 57.34675 103.95575) (end 61.51475 103.95575) (width 0.381) (layer B.Cu) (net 9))
 (segment (start 56.03875 102.64775) (end 57.34675 103.95575) (width 0.381) (layer B.Cu) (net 9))
 (segment (start 57.15 101.5365) (end 56.03875 102.64775) (width 0.381) (layer B.Cu) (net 9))
 (segment (start 57.15 99.21875) (end 57.15 101.5365) (width 0.381) (layer B.Cu) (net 9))
 (segment (start 65.61475 98.383652) (end 65.61475 97.45575) (width 0.381) (layer B.Cu) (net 9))
 (segment (start 66.386848 99.15575) (end 65.61475 98.383652) (width 0.381) (layer B.Cu) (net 9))
 (segment (start 72.91475 99.15575) (end 66.386848 99.15575) (width 0.381) (layer B.Cu) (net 9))
 (segment (start 64.01475 105.527848) (end 62.442652 103.95575) (width 0.381) (layer B.Cu) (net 9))
 (segment (start 62.442652 103.95575) (end 61.51475 103.95575) (width 0.381) (layer B.Cu) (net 9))
 (segment (start 64.01475 108.85575) (end 64.01475 105.527848) (width 0.381) (layer B.Cu) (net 9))
 (segment (start 70.41475 112.9415) (end 70.41475 108.85575) (width 0.381) (layer B.Cu) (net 9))
 (segment (start 69.05625 114.3) (end 70.41475 112.9415) (width 0.381) (layer B.Cu) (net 9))
 (segment (start 64.01475 113.84875) (end 64.01475 108.85575) (width 0.381) (layer B.Cu) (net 9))
 (segment (start 63.78575 114.07775) (end 64.01475 113.84875) (width 0.381) (layer B.Cu) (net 9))
 (segment (start 64.008 114.3) (end 63.78575 114.07775) (width 0.381) (layer B.Cu) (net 9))
 (segment (start 69.05625 114.3) (end 64.008 114.3) (width 0.381) (layer B.Cu) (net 9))
 (segment (start 71.802151 107.715249) (end 70.627349 107.715249) (width 0.381) (layer B.Cu) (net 9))
 (segment (start 70.41475 107.927848) (end 70.41475 108.85575) (width 0.381) (layer B.Cu) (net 9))
 (segment (start 70.627349 107.715249) (end 70.41475 107.927848) (width 0.381) (layer B.Cu) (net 9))
 (segment (start 72.949402 108.8625) (end 71.802151 107.715249) (width 0.381) (layer B.Cu) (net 9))
 (segment (start 76.2 108.8625) (end 72.949402 108.8625) (width 0.381) (layer B.Cu) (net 9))
 (segment (start 50.01875 86.9685) (end 55.284 92.23375) (width 0.381) (layer B.Cu) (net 9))
 (segment (start 55.284 92.23375) (end 61.2775 92.23375) (width 0.381) (layer B.Cu) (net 9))
 (segment (start 50.01875 85.4625) (end 50.01875 86.9685) (width 0.381) (layer B.Cu) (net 9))
 (segment (start 43.73125 113.76875) (end 42.33125 113.76875) (width 0.381) (layer B.Cu) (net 9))
 (segment (start 42.33125 113.76875) (end 42.33125 108.48125) (width 0.381) (layer B.Cu) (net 9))
 (segment (start 42.33125 108.48125) (end 42.8625 107.95) (width 0.381) (layer B.Cu) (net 9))
 (via (at 50.8 107.95) (size 0.8) (drill 0.4) (layers F.Cu B.Cu) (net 9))
 (segment (start 42.8625 107.95) (end 50.8 107.95) (width 0.381) (layer B.Cu) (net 9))
 (via (at 55.814058 102.935942) (size 0.8) (drill 0.4) (layers F.Cu B.Cu) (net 9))
 (segment (start 50.8 107.95) (end 55.814058 102.935942) (width 0.381) (layer F.Cu) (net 9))
 (via (at 60.164748 103.88275) (size 0.8) (drill 0.4) (layers F.Cu B.Cu) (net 9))
 (segment (start 60.237748 103.95575) (end 60.164748 103.88275) (width 0.381) (layer B.Cu) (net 9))
 (segment (start 61.51475 103.95575) (end 60.237748 103.95575) (width 0.381) (layer B.Cu) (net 9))
 (segment (start 60.164748 103.88275) (end 64.29375 99.753748) (width 0.381) (layer F.Cu) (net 9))
 (via (at 64.369118 95.968382) (size 0.8) (drill 0.4) (layers F.Cu B.Cu) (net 9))
 (segment (start 64.29375 96.04375) (end 64.369118 95.968382) (width 0.381) (layer F.Cu) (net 9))
 (segment (start 64.29375 99.753748) (end 64.29375 96.04375) (width 0.381) (layer F.Cu) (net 9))
 (segment (start 65.009116 95.968382) (end 65.61475 96.574016) (width 0.381) (layer B.Cu) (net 9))
 (segment (start 65.61475 96.574016) (end 65.61475 97.45575) (width 0.381) (layer B.Cu) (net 9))
 (segment (start 64.369118 95.968382) (end 65.009116 95.968382) (width 0.381) (layer B.Cu) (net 9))
 (via (at 65.88125 93.6625) (size 0.8) (drill 0.4) (layers F.Cu B.Cu) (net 9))
 (segment (start 65.73375 93.515) (end 65.88125 93.6625) (width 0.381) (layer B.Cu) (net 9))
 (segment (start 65.73375 92.10675) (end 65.73375 93.515) (width 0.381) (layer B.Cu) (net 9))
 (segment (start 65.88125 94.45625) (end 64.369118 95.968382) (width 0.381) (layer F.Cu) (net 9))
 (segment (start 65.88125 93.6625) (end 65.88125 94.45625) (width 0.381) (layer F.Cu) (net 9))
 (segment (start 75.69875 99.95575) (end 72.91475 99.95575) (width 0.381) (layer B.Cu) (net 10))
 (segment (start 76.41975 100.67675) (end 75.69875 99.95575) (width 0.381) (layer B.Cu) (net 10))
 (segment (start 60.586848 102.35575) (end 61.51475 102.35575) (width 0.381) (layer B.Cu) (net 10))
 (segment (start 60.374249 102.143151) (end 60.586848 102.35575) (width 0.381) (layer B.Cu) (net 10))
 (segment (start 60.374249 100.542999) (end 60.374249 102.143151) (width 0.381) (layer B.Cu) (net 10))
 (segment (start 57.15 97.31875) (end 60.374249 100.542999) (width 0.381) (layer B.Cu) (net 10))
 (segment (start 66.18375 99.95575) (end 64.81475 98.58675) (width 0.381) (layer B.Cu) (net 10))
 (segment (start 72.91475 99.95575) (end 66.18375 99.95575) (width 0.381) (layer B.Cu) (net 10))
 (segment (start 62.442652 106.35575) (end 61.51475 106.35575) (width 0.381) (layer B.Cu) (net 10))
 (segment (start 63.21475 107.127848) (end 62.442652 106.35575) (width 0.381) (layer B.Cu) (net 10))
 (segment (start 63.21475 108.85575) (end 63.21475 107.127848) (width 0.381) (layer B.Cu) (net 10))
 (segment (start 62.64575 102.35575) (end 64.81475 100.18675) (width 0.381) (layer B.Cu) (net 10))
 (segment (start 64.81475 100.18675) (end 64.81475 98.15225) (width 0.381) (layer B.Cu) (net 10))
 (segment (start 61.51475 102.35575) (end 62.64575 102.35575) (width 0.381) (layer B.Cu) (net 10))
 (segment (start 64.81475 98.15225) (end 64.81475 97.45575) (width 0.381) (layer B.Cu) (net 10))
 (segment (start 64.81475 98.58675) (end 64.81475 98.15225) (width 0.381) (layer B.Cu) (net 10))
 (segment (start 71.21475 114.0415) (end 71.21475 108.85575) (width 0.381) (layer B.Cu) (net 10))
 (segment (start 70.95625 114.3) (end 71.21475 114.0415) (width 0.381) (layer B.Cu) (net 10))
 (segment (start 61.88575 110.18475) (end 63.21475 108.85575) (width 0.381) (layer B.Cu) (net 10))
 (segment (start 61.88575 114.07775) (end 61.88575 110.18475) (width 0.381) (layer B.Cu) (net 10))
 (segment (start 57.15 93.472) (end 57.05475 93.37675) (width 0.381) (layer B.Cu) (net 10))
 (segment (start 57.15 97.31875) (end 57.15 93.472) (width 0.381) (layer B.Cu) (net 10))
 (via (at 46.0375 93.6625) (size 0.8) (drill 0.4) (layers F.Cu B.Cu) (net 10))
 (segment (start 44.45 93.6625) (end 46.0375 93.6625) (width 0.381) (layer B.Cu) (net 10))
 (segment (start 46.0375 93.6625) (end 55.5625 93.6625) (width 0.381) (layer F.Cu) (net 10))
 (via (at 55.5625 93.6625) (size 0.8) (drill 0.4) (layers F.Cu B.Cu) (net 10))
 (segment (start 56.769 93.6625) (end 57.05475 93.37675) (width 0.381) (layer B.Cu) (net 10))
 (segment (start 55.5625 93.6625) (end 56.769 93.6625) (width 0.381) (layer B.Cu) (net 10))
 (segment (start 63.22351 115.41551) (end 61.88575 114.07775) (width 0.381) (layer B.Cu) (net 10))
 (segment (start 69.84074 115.41551) (end 63.22351 115.41551) (width 0.381) (layer B.Cu) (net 10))
 (segment (start 70.95625 114.3) (end 69.84074 115.41551) (width 0.381) (layer B.Cu) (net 10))
 (via (at 59.53125 106.3625) (size 0.8) (drill 0.4) (layers F.Cu B.Cu) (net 10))
 (segment (start 59.538 106.35575) (end 59.53125 106.3625) (width 0.381) (layer B.Cu) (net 10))
 (segment (start 61.51475 106.35575) (end 59.538 106.35575) (width 0.381) (layer B.Cu) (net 10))
 (via (at 59.53125 102.39375) (size 0.8) (drill 0.4) (layers F.Cu B.Cu) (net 10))
 (segment (start 59.131251 102.793749) (end 59.53125 102.39375) (width 0.381) (layer F.Cu) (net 10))
 (segment (start 59.131251 105.962501) (end 59.131251 102.793749) (width 0.381) (layer F.Cu) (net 10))
 (segment (start 59.53125 106.3625) (end 59.131251 105.962501) (width 0.381) (layer F.Cu) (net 10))
 (segment (start 60.548848 102.39375) (end 60.586848 102.35575) (width 0.381) (layer B.Cu) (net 10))
 (segment (start 59.53125 102.39375) (end 60.548848 102.39375) (width 0.381) (layer B.Cu) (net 10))
 (segment (start 62.20775 90.40675) (end 62.13475 90.33375) (width 0.254) (layer B.Cu) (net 2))
 (segment (start 65.73375 90.40675) (end 62.20775 90.40675) (width 0.254) (layer B.Cu) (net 2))
 (segment (start 58.44675 103.15575) (end 61.51475 103.15575) (width 0.254) (layer B.Cu) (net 38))
 (segment (start 57.93875 102.64775) (end 58.44675 103.15575) (width 0.254) (layer B.Cu) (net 38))
 (segment (start 94.25 87.25) (end 91.4 84.4) (width 0.254) (layer B.Cu) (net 45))
 (segment (start 96.8375 87.25) (end 94.25 87.25) (width 0.254) (layer B.Cu) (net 45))
 (segment (start 97.764501 108.672999) (end 96.8375 109.6) (width 0.254) (layer B.Cu) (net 22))
 (segment (start 97.764501 91.477001) (end 97.764501 108.672999) (width 0.254) (layer B.Cu) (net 22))
 (segment (start 96.8375 90.55) (end 97.764501 91.477001) (width 0.254) (layer B.Cu) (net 22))
 (segment (start 96.166599 110.270901) (end 96.8375 109.6) (width 0.254) (layer B.Cu) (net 22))
 (segment (start 84.361939 110.270901) (end 96.166599 110.270901) (width 0.254) (layer B.Cu) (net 22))
 (segment (start 78.046788 103.95575) (end 84.361939 110.270901) (width 0.254) (layer B.Cu) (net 22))
 (segment (start 72.91475 103.95575) (end 78.046788 103.95575) (width 0.254) (layer B.Cu) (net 22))
 (segment (start 113.3 87.25) (end 110.45 84.4) (width 0.254) (layer B.Cu) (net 44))
 (segment (start 115.8875 87.25) (end 113.3 87.25) (width 0.254) (layer B.Cu) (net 44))
 (segment (start 116.814501 91.477001) (end 115.8875 90.55) (width 0.254) (layer B.Cu) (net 21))
 (segment (start 116.814501 107.968999) (end 116.814501 91.477001) (width 0.254) (layer B.Cu) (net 21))
 (segment (start 115.8875 108.896) (end 116.814501 107.968999) (width 0.254) (layer B.Cu) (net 21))
 (segment (start 115.8875 109.6) (end 115.8875 108.896) (width 0.254) (layer B.Cu) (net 21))
 (segment (start 84.173882 110.724911) (end 114.762589 110.724911) (width 0.254) (layer B.Cu) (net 21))
 (segment (start 78.204722 104.75575) (end 84.173882 110.724911) (width 0.254) (layer B.Cu) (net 21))
 (segment (start 114.762589 110.724911) (end 115.8875 109.6) (width 0.254) (layer B.Cu) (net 21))
 (segment (start 72.91475 104.75575) (end 78.204722 104.75575) (width 0.254) (layer B.Cu) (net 21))
 (segment (start 94.25 106.3) (end 91.4 103.45) (width 0.254) (layer B.Cu) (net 43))
 (segment (start 96.8375 106.3) (end 94.25 106.3) (width 0.254) (layer B.Cu) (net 43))
 (segment (start 113.8625 106.3) (end 110.49 102.9275) (width 0.254) (layer B.Cu) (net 42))
 (segment (start 115.8875 106.3) (end 113.8625 106.3) (width 0.254) (layer B.Cu) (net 42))
 (segment (start 85.09 86.36) (end 104.14 86.36) (width 0.254) (layer F.Cu) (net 24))
 (segment (start 76.281768 102.35575) (end 85.09 93.547518) (width 0.254) (layer B.Cu) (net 24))
 (segment (start 85.09 93.547518) (end 85.09 86.36) (width 0.254) (layer B.Cu) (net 24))
 (segment (start 72.91475 102.35575) (end 76.281768 102.35575) (width 0.254) (layer B.Cu) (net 24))
 (segment (start 104.0825 105.41) (end 104.14 105.4675) (width 0.254) (layer F.Cu) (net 23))
 (segment (start 85.09 105.41) (end 104.0825 105.41) (width 0.254) (layer F.Cu) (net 23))
 (segment (start 82.83575 103.15575) (end 85.09 105.41) (width 0.254) (layer B.Cu) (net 23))
 (segment (start 72.91475 103.15575) (end 82.83575 103.15575) (width 0.254) (layer B.Cu) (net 23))
 (segment (start 60.749352 93.37675) (end 64.01475 96.642148) (width 0.254) (layer B.Cu) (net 32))
 (segment (start 58.87975 93.37675) (end 60.749352 93.37675) (width 0.254) (layer B.Cu) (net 32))
 (via (at 51.59375 108.74375) (size 0.8) (drill 0.4) (layers F.Cu B.Cu) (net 32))
 (segment (start 50.26875 110.06875) (end 51.59375 108.74375) (width 0.254) (layer B.Cu) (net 32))
 (segment (start 49.93125 110.06875) (end 50.26875 110.06875) (width 0.254) (layer B.Cu) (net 32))
 (segment (start 51.59375 108.74375) (end 58.7375 101.6) (width 0.254) (layer F.Cu) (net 32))
 (segment (start 58.7375 101.6) (end 58.7375 97.63125) (width 0.254) (layer F.Cu) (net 32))
 (segment (start 58.7375 97.63125) (end 60.325 96.04375) (width 0.254) (layer F.Cu) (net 32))
 (via (at 62.70625 96.04375) (size 0.8) (drill 0.4) (layers F.Cu B.Cu) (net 32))
 (segment (start 60.325 96.04375) (end 62.70625 96.04375) (width 0.254) (layer F.Cu) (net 32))
 (segment (start 64.01475 96.642148) (end 64.01475 97.45575) (width 0.254) (layer B.Cu) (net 32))
 (segment (start 63.416352 96.04375) (end 64.01475 96.642148) (width 0.254) (layer B.Cu) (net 32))
 (segment (start 62.70625 96.04375) (end 63.416352 96.04375) (width 0.254) (layer B.Cu) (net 32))
 (segment (start 73.033 107.0375) (end 72.91475 107.15575) (width 0.254) (layer B.Cu) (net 18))
 (segment (start 76.2 107.0375) (end 73.033 107.0375) (width 0.254) (layer B.Cu) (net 18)))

